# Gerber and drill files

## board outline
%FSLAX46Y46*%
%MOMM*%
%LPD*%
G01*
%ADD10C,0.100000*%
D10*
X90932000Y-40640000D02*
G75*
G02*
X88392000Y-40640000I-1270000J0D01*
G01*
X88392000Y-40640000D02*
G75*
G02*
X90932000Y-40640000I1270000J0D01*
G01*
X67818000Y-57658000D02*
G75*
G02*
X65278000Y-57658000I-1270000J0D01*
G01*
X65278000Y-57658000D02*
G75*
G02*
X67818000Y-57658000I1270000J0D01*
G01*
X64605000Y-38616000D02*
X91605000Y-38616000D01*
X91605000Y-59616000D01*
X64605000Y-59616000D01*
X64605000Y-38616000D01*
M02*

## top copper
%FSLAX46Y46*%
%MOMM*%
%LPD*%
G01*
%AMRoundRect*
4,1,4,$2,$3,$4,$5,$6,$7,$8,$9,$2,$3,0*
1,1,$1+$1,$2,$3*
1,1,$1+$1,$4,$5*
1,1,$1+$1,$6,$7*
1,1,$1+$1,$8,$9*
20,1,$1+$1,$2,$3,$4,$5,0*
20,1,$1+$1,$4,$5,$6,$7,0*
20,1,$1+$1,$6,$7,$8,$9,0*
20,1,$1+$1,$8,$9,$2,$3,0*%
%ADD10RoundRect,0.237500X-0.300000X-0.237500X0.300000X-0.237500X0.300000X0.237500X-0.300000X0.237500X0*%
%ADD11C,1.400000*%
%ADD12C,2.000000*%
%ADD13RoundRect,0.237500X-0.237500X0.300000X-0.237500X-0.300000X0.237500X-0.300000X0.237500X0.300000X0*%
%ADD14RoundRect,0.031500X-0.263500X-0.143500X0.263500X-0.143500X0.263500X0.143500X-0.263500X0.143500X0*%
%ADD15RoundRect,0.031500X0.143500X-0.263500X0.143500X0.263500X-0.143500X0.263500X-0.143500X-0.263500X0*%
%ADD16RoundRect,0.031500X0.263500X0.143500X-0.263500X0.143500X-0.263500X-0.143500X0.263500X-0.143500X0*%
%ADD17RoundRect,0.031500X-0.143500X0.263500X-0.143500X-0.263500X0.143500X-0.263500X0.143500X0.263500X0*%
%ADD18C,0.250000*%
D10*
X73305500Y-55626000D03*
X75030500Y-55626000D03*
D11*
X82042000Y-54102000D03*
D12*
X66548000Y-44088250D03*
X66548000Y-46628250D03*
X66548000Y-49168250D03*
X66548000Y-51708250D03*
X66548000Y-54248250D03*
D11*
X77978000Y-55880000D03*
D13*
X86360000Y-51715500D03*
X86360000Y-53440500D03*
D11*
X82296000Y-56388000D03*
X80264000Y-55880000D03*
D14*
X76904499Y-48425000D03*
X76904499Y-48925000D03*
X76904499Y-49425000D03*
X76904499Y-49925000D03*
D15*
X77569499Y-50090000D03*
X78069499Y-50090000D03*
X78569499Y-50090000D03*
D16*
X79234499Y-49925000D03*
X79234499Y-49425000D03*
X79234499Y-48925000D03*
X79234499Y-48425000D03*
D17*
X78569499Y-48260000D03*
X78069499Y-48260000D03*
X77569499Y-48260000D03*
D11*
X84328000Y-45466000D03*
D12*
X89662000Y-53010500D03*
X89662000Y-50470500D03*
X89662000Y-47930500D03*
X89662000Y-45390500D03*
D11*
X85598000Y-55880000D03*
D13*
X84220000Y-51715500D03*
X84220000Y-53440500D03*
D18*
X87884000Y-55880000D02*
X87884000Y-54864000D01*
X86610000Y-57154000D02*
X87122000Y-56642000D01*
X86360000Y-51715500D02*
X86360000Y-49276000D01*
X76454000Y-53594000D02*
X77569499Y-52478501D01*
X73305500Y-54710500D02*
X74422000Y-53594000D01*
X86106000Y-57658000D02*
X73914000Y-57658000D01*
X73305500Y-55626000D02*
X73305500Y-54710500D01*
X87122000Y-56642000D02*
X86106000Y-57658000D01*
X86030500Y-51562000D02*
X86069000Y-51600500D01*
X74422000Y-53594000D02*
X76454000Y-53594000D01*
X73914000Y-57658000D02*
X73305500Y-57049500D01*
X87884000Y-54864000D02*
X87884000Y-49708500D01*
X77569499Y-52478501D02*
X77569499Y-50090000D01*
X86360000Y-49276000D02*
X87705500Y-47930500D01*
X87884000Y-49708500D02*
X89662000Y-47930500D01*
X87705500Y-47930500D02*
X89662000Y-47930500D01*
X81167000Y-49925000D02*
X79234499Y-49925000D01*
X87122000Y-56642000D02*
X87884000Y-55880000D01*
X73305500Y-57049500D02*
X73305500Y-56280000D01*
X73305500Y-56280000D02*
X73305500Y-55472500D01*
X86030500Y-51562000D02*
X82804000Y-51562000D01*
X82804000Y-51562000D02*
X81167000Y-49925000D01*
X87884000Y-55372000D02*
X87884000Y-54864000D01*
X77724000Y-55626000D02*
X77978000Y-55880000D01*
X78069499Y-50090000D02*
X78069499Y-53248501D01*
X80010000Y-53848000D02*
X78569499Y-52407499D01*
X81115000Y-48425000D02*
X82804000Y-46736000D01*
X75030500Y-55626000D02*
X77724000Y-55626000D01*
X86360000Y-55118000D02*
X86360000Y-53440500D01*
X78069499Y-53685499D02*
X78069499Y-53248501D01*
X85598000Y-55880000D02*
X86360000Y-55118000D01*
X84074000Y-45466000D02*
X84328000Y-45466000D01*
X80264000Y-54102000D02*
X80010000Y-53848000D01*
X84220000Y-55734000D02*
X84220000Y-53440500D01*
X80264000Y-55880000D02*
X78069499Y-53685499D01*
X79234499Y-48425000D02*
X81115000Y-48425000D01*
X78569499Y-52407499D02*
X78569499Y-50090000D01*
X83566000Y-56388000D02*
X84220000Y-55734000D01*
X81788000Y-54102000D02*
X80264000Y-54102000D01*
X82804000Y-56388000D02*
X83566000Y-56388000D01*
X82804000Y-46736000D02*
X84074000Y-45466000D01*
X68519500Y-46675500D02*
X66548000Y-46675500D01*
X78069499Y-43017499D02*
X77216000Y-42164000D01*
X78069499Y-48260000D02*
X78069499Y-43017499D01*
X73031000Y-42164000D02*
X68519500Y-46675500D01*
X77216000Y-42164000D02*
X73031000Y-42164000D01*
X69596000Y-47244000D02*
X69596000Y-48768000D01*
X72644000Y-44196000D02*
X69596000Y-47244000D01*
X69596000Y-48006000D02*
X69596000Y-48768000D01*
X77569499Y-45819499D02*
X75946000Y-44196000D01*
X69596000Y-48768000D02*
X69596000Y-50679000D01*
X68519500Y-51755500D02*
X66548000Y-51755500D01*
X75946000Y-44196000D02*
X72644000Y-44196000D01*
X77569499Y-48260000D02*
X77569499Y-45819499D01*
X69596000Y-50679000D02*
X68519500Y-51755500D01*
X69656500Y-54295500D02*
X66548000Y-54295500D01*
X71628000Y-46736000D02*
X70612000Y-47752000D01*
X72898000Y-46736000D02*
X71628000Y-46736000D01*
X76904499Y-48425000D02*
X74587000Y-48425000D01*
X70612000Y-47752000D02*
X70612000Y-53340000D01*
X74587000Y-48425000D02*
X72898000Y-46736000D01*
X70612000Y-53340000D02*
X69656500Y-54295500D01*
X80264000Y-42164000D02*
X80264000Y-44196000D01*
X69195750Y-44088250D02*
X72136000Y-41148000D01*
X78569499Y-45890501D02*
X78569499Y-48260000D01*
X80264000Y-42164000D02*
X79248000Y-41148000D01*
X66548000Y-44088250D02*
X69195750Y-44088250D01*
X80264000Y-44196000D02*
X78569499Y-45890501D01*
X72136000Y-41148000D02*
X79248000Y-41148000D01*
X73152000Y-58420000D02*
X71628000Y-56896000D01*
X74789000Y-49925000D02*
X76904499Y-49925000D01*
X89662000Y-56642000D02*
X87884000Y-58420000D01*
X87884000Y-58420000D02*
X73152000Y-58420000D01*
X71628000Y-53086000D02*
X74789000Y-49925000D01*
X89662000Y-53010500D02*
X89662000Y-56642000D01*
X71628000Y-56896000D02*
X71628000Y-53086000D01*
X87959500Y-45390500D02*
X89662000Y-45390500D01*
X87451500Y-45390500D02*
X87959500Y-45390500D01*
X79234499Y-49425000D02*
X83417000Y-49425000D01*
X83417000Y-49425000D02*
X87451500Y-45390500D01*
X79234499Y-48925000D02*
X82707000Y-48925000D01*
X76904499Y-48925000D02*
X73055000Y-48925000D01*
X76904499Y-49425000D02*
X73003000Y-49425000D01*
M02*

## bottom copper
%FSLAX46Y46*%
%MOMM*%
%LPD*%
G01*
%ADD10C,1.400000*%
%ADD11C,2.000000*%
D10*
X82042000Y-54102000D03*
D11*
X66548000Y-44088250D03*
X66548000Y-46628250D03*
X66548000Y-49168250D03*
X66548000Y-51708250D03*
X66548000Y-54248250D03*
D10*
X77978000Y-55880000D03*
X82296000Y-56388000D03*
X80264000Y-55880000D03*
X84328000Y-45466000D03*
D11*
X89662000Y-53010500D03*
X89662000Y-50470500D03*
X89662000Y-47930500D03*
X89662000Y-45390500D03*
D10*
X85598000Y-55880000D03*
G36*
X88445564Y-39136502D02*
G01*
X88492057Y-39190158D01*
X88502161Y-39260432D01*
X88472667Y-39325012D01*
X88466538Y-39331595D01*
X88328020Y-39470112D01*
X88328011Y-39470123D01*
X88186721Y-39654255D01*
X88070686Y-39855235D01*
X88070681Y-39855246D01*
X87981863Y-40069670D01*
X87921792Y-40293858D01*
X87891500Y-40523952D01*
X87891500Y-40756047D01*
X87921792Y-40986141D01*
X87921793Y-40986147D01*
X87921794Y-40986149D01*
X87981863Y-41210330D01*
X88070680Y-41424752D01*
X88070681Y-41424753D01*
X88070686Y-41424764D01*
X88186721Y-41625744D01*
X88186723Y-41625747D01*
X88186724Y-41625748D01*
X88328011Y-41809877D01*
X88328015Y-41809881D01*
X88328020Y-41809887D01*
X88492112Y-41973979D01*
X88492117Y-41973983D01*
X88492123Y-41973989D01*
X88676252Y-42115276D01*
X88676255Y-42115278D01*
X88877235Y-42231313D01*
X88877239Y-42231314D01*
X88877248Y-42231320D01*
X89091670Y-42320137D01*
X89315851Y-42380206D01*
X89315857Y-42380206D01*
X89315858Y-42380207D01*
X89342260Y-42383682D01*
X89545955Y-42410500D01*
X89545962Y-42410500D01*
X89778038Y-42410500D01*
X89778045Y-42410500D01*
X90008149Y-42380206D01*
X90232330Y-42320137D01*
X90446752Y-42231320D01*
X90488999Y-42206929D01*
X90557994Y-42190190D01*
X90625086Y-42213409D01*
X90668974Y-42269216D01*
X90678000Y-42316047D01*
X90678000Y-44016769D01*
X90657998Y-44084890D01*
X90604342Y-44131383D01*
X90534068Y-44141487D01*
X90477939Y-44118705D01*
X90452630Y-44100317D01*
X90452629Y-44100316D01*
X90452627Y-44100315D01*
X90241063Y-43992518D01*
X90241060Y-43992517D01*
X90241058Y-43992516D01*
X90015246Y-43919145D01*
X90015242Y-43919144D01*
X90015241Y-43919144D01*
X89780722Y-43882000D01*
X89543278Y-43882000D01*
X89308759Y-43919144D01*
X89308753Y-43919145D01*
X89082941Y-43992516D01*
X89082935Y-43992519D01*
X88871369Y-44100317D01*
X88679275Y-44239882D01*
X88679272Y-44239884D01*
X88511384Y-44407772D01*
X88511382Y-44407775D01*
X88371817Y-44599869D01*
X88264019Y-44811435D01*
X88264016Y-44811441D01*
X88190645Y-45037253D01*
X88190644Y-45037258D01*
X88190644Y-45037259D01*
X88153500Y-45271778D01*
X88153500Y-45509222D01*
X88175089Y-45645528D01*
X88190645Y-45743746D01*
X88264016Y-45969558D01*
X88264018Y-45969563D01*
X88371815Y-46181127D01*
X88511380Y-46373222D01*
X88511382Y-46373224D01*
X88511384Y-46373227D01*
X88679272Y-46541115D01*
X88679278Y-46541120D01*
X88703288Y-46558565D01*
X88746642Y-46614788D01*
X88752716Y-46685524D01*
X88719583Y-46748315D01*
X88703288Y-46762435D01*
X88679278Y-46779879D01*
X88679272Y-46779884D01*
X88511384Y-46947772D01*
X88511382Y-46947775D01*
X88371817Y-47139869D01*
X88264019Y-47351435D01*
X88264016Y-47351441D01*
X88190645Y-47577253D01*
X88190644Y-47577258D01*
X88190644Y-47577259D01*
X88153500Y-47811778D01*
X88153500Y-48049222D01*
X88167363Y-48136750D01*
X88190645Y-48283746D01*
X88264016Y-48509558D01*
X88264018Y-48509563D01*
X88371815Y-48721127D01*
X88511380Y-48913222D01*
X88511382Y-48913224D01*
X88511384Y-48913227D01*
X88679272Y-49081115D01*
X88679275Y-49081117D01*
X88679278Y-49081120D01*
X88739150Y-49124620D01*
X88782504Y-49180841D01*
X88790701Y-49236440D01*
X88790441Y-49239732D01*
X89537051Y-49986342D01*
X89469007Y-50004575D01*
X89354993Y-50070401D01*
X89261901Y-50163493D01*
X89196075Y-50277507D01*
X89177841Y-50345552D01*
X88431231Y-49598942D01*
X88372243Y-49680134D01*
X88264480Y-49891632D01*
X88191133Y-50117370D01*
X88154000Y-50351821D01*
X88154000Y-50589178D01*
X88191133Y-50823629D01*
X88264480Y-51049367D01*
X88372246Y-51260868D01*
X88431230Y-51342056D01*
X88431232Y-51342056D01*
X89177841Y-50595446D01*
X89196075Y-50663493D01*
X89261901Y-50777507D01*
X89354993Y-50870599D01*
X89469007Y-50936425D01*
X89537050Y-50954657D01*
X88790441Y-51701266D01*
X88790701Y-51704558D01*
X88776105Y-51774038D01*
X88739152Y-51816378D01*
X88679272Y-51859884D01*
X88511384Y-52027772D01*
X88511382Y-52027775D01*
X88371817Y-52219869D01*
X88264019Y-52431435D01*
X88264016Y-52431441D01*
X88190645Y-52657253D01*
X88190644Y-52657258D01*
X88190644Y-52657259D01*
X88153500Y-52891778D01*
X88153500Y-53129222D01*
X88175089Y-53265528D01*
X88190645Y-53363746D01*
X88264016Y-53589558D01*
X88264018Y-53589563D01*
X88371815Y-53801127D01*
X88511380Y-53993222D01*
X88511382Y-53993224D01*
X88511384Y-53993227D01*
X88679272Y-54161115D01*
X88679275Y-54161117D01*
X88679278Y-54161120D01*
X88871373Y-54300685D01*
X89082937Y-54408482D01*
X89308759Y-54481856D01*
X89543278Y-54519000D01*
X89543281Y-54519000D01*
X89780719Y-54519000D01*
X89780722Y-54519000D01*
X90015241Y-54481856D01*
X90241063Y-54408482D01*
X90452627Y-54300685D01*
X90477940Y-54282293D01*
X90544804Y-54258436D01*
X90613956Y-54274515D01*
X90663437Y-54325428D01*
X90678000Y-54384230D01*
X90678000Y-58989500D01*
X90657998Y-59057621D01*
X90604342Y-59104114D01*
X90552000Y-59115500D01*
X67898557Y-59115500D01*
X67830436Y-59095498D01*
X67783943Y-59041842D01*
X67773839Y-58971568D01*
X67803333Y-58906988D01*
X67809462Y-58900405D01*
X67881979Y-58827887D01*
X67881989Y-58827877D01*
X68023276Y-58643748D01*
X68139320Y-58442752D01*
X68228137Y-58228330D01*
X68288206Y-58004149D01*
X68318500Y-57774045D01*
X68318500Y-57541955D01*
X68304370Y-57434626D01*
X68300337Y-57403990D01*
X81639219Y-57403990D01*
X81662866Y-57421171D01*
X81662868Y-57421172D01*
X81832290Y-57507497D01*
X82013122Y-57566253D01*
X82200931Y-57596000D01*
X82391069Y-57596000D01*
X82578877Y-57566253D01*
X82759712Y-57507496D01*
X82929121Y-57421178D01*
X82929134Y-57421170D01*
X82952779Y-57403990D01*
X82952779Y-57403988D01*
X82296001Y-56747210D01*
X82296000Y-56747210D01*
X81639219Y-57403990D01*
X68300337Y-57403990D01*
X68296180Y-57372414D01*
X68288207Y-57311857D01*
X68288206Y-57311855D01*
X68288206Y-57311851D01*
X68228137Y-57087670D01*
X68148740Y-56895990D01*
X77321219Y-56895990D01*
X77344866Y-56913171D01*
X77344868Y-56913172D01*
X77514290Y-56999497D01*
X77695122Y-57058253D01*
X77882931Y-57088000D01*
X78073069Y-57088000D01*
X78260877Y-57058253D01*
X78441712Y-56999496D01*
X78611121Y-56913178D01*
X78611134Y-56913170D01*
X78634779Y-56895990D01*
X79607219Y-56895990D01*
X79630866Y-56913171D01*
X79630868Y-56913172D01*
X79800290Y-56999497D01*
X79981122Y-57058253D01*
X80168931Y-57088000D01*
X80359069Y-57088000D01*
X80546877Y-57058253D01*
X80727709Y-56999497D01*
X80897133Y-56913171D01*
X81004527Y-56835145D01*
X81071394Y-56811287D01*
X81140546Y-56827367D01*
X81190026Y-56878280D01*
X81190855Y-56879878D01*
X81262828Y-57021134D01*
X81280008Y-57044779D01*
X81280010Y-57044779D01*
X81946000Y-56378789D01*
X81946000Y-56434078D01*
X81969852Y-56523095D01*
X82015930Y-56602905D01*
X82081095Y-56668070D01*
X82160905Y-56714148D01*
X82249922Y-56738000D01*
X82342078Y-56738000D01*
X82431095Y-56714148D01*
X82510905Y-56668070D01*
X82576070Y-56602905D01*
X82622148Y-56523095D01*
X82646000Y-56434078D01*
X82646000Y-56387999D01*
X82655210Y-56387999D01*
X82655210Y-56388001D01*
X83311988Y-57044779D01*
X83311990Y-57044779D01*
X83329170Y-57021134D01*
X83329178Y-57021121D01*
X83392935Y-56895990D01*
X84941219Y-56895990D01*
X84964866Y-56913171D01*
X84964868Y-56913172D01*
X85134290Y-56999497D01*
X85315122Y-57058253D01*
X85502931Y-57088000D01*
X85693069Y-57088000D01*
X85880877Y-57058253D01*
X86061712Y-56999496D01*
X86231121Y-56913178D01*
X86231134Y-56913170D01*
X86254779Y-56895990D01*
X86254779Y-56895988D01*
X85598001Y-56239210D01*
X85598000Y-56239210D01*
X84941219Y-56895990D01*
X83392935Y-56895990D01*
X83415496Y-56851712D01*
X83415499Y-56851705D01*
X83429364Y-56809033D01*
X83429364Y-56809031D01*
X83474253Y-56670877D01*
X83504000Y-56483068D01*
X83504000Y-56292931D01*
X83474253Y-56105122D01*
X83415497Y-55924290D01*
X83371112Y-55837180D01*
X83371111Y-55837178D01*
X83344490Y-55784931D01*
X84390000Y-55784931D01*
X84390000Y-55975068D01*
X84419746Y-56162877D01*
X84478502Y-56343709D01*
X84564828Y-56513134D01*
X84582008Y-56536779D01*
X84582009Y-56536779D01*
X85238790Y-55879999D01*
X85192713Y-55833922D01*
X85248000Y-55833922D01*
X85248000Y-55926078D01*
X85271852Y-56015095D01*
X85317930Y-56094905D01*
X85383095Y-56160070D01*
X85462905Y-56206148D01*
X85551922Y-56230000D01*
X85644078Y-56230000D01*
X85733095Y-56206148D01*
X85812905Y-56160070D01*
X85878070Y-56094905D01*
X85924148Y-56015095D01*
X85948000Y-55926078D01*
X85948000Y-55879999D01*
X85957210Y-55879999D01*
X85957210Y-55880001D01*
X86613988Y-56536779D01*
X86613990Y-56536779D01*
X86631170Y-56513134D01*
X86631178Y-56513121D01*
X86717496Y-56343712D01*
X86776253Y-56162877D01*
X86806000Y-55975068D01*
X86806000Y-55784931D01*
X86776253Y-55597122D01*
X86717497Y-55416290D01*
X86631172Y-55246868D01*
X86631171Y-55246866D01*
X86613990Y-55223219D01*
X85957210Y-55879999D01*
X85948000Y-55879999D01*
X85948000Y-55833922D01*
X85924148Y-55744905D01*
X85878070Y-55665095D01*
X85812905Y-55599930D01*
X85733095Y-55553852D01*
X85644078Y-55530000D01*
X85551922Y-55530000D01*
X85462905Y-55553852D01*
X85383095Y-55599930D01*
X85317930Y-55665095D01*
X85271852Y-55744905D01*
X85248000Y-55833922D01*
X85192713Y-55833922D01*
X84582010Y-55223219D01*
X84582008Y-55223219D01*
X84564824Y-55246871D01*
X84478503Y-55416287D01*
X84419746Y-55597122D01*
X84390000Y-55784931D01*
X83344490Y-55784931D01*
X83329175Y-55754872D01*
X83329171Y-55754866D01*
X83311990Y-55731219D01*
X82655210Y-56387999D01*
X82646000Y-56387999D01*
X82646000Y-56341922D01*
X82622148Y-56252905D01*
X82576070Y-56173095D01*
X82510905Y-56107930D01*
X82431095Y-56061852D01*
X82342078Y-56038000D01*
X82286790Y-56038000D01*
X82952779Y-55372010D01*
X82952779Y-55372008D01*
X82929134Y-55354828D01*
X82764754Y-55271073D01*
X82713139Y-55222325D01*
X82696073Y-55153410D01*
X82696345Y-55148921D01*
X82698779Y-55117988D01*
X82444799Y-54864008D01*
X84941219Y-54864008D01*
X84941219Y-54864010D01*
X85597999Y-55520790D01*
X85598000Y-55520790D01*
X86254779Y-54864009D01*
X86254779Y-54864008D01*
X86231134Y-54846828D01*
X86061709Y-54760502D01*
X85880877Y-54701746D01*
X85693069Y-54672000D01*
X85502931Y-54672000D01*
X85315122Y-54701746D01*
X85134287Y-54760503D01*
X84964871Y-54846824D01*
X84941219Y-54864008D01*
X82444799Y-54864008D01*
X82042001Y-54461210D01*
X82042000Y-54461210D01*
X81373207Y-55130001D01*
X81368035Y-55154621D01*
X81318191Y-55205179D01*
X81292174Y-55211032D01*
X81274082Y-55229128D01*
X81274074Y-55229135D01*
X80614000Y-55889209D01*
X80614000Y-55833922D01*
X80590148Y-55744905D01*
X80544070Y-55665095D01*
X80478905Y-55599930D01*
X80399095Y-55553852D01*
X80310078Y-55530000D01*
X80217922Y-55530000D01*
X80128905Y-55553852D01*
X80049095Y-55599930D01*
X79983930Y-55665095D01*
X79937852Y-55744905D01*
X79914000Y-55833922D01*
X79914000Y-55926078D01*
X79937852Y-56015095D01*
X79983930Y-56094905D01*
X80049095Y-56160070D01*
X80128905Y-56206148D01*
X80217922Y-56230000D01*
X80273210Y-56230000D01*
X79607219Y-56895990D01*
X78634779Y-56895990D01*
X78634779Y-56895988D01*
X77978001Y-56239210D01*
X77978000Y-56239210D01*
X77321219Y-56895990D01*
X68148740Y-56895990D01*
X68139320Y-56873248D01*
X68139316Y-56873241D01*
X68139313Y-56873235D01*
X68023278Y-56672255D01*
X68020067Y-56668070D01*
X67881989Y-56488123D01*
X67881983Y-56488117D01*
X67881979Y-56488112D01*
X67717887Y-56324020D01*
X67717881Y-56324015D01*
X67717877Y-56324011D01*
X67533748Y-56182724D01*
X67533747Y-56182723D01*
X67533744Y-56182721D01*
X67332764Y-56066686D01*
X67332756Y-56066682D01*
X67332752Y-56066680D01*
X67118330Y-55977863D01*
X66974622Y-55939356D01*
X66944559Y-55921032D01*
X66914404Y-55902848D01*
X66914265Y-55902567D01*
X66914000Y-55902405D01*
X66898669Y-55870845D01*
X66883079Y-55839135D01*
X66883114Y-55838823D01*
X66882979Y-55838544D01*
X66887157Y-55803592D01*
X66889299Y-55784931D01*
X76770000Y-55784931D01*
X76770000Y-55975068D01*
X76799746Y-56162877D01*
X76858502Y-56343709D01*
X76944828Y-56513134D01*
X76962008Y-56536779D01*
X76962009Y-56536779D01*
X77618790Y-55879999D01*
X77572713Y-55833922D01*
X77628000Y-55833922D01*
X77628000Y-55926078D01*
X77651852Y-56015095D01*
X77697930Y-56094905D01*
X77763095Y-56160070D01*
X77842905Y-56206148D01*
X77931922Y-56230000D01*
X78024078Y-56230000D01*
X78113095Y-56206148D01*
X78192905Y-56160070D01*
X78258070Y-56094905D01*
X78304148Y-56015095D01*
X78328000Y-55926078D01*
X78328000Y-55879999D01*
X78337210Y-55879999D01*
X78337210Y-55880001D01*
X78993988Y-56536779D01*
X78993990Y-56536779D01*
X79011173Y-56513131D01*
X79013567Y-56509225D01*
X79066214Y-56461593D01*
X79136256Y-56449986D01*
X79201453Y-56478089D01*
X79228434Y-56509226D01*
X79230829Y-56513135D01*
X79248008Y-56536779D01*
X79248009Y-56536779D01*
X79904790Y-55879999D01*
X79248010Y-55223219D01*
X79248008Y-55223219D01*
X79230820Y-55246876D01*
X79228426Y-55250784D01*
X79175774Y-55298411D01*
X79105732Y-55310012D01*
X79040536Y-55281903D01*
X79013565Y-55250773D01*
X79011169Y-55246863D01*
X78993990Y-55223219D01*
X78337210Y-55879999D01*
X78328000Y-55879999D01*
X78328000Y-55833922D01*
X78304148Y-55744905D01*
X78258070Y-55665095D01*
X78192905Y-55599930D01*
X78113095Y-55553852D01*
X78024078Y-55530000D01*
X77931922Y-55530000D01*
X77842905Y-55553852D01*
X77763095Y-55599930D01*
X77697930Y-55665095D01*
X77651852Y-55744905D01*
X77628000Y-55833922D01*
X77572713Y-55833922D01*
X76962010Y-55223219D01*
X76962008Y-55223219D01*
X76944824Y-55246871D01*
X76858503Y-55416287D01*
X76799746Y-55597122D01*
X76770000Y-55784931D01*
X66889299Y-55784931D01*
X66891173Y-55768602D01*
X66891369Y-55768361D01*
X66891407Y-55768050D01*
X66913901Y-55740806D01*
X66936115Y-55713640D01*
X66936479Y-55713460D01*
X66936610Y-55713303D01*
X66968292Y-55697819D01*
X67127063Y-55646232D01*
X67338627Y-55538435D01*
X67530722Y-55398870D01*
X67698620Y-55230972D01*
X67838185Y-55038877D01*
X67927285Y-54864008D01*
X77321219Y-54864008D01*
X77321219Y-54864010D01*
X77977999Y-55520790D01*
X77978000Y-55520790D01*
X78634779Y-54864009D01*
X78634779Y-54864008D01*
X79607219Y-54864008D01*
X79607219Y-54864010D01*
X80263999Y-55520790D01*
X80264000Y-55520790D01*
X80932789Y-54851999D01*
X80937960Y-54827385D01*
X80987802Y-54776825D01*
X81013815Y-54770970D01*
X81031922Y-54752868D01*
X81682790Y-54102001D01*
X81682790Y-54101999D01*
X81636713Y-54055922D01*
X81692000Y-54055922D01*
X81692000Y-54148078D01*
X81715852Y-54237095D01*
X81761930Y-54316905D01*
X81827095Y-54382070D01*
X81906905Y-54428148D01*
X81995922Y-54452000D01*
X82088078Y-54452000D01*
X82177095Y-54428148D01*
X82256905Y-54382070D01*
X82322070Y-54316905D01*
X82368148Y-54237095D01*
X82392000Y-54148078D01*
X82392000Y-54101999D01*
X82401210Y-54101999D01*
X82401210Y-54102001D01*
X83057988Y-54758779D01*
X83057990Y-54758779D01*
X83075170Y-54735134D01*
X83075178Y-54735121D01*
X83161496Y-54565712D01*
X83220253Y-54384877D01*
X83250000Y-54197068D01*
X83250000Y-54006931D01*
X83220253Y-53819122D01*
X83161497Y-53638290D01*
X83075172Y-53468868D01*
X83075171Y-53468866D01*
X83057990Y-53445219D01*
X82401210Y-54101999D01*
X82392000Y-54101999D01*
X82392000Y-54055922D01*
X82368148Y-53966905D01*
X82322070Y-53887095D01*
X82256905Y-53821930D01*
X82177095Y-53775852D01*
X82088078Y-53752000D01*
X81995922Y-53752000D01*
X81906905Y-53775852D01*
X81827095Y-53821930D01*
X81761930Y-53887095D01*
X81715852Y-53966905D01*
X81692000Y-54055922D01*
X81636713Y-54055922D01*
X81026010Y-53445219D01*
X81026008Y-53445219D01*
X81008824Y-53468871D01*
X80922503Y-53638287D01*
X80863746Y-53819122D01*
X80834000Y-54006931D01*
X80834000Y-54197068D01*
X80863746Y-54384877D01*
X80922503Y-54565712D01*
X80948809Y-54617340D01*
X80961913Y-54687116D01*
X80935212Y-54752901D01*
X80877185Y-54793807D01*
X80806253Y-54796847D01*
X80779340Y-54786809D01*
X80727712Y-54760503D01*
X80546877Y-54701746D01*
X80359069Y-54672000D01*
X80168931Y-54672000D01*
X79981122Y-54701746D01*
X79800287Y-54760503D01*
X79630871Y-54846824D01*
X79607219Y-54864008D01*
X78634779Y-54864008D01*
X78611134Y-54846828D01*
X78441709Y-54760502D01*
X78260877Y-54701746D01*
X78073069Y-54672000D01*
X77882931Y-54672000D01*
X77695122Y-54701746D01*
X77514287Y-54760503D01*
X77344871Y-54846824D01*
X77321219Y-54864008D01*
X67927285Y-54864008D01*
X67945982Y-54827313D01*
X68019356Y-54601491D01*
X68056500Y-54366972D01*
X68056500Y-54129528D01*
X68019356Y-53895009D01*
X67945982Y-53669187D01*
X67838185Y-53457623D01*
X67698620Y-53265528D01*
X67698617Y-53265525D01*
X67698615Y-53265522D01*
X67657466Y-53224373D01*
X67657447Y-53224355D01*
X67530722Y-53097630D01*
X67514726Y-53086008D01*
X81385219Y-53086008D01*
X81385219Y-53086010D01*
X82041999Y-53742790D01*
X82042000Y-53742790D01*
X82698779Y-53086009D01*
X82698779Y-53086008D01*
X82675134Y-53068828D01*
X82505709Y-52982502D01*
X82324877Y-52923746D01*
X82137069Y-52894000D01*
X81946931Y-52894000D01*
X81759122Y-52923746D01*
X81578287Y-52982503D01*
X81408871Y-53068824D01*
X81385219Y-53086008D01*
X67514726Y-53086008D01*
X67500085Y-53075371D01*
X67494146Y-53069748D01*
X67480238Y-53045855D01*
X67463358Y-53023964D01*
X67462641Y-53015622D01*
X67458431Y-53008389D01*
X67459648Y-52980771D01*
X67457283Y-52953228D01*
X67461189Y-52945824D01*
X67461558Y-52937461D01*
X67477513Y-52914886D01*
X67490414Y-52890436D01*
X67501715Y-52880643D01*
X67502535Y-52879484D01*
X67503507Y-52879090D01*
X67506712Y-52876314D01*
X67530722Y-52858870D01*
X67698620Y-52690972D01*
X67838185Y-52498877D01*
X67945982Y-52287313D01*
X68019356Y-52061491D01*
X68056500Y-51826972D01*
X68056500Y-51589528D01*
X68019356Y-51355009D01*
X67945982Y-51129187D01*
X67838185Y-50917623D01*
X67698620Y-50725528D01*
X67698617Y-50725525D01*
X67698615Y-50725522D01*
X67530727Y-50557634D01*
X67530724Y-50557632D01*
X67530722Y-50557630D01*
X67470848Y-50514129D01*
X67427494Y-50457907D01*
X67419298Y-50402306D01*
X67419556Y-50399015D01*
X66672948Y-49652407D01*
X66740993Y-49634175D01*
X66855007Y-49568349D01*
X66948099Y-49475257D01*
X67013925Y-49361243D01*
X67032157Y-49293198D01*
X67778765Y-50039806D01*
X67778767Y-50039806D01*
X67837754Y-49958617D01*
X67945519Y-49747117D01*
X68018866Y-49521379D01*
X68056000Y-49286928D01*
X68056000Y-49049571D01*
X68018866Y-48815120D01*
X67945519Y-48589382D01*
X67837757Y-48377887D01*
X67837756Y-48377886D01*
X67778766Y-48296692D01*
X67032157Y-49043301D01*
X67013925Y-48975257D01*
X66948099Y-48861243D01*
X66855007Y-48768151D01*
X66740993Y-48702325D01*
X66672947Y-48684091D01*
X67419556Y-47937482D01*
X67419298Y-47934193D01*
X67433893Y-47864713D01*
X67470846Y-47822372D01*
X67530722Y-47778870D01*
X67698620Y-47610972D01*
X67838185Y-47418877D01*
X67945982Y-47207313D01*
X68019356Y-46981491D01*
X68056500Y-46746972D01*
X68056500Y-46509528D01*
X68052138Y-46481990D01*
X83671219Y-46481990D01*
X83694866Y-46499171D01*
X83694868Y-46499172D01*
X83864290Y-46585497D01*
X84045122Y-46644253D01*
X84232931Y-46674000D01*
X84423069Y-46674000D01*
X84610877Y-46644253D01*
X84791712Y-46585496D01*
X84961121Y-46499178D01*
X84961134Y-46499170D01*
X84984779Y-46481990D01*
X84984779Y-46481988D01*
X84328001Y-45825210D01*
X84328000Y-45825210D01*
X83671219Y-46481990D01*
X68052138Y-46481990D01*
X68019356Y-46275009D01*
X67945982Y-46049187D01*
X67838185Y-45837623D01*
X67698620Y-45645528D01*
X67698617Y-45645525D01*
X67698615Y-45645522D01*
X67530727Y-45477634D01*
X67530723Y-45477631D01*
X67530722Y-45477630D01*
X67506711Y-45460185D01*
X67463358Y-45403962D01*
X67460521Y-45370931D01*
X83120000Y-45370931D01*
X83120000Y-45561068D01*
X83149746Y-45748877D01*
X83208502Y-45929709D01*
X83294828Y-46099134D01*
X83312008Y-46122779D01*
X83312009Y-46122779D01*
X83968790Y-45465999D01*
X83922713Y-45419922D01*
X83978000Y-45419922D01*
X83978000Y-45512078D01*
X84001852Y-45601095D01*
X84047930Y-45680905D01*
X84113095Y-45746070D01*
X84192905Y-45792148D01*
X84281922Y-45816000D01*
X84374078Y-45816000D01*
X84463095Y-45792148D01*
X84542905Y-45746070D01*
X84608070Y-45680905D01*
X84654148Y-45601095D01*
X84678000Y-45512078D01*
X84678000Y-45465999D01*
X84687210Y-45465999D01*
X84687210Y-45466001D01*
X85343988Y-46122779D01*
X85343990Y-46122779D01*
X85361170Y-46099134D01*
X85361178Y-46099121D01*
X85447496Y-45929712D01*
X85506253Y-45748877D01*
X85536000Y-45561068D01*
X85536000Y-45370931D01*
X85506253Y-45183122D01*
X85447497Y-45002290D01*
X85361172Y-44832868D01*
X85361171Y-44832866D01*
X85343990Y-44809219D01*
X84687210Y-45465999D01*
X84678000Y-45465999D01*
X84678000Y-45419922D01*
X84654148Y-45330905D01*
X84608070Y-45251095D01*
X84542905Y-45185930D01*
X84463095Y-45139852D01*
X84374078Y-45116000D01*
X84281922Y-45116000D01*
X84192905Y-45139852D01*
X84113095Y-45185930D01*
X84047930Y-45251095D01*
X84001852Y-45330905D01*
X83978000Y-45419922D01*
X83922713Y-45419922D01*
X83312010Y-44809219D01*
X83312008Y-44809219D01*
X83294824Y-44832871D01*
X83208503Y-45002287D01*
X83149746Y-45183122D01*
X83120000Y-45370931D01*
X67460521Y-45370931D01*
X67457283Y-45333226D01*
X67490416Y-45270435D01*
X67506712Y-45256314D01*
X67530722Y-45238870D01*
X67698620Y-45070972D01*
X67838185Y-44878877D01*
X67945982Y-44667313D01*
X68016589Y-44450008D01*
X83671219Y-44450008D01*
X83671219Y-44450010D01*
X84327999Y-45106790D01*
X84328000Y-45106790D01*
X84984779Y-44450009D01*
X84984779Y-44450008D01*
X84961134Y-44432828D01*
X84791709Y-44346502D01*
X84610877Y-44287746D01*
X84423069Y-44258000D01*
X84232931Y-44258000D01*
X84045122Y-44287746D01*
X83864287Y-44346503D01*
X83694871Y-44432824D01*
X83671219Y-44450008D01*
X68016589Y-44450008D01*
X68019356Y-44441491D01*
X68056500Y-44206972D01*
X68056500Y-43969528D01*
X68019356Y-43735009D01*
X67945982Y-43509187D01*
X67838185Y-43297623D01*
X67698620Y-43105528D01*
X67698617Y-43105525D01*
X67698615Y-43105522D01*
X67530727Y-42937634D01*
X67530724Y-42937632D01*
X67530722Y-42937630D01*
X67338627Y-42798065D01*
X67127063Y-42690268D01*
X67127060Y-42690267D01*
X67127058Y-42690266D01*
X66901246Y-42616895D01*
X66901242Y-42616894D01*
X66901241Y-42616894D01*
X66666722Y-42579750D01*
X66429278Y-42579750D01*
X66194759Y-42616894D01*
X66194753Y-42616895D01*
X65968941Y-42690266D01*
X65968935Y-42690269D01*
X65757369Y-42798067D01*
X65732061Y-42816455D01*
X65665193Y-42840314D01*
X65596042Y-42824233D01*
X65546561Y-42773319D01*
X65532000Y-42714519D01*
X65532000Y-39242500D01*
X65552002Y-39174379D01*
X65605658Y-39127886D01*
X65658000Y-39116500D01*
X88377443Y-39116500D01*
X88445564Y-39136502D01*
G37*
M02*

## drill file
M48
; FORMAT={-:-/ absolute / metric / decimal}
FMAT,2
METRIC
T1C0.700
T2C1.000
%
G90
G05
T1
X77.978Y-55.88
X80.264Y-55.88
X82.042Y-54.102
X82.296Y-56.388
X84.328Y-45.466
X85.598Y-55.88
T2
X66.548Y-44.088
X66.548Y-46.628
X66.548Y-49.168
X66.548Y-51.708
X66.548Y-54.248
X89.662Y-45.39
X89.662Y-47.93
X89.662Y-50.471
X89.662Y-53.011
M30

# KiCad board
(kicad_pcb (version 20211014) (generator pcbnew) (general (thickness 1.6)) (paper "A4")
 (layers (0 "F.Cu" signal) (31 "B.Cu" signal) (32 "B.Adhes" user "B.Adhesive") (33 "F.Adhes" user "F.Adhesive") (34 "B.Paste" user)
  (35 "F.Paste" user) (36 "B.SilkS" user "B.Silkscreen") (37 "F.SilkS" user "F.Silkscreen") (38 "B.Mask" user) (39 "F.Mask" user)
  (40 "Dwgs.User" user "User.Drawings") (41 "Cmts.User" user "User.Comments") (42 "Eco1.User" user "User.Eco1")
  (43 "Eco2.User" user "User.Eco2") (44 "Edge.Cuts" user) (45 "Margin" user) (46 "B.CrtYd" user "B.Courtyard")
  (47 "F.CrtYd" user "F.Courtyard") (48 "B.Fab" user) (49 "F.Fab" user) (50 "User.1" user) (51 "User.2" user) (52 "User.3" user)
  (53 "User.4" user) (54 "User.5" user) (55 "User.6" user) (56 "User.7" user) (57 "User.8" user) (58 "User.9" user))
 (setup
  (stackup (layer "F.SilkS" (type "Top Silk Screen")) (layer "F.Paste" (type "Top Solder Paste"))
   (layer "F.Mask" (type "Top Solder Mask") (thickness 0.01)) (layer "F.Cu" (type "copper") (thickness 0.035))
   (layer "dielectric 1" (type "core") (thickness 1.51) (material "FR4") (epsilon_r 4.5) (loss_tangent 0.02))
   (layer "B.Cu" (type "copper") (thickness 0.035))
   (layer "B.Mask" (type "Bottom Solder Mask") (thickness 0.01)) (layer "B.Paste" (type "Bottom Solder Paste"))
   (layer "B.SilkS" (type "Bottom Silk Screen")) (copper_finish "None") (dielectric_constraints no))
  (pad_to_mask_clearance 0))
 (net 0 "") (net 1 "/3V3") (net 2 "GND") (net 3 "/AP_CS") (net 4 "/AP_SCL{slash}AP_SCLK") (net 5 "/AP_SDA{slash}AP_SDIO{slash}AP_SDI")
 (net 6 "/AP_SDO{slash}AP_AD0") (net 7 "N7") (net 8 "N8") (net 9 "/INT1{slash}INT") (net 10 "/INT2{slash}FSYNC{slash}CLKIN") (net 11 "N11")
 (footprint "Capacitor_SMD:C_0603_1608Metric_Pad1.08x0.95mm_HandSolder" (layer "F.Cu") (at 74.168 55.626)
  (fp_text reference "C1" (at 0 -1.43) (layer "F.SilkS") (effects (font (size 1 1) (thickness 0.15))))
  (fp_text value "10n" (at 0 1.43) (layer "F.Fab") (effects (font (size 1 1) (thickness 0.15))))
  (pad "1" smd roundrect (at -0.8625 0) (size 1.075 0.95) (layers "F.Cu" "F.Paste" "F.Mask") (roundrect_rratio 0.25) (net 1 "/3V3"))
  (pad "2" smd roundrect (at 0.8625 0) (size 1.075 0.95) (layers "F.Cu" "F.Paste" "F.Mask") (roundrect_rratio 0.25) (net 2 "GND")))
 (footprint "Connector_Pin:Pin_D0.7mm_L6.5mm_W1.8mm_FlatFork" (layer "F.Cu") (at 82.042 54.102)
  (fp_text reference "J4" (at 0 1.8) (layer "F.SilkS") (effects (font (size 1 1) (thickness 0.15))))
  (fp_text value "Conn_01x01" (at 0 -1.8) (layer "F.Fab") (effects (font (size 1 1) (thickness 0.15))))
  (pad "1" thru_hole circle (at 0 0) (size 1.4 1.4) (drill 0.7) (layers *.Cu *.Mask) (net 2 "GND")))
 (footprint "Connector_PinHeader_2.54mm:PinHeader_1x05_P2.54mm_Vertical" (layer "F.Cu") (at 66.548 44.08825)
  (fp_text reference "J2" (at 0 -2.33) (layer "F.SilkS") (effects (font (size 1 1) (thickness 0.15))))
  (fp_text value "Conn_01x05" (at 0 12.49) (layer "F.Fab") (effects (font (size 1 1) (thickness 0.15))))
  (pad "1" thru_hole circle (at 0 0) (size 2 2) (drill 1) (layers *.Cu *.Mask) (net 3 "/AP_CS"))
  (pad "2" thru_hole circle (at 0 2.54) (size 2 2) (drill 1) (layers *.Cu *.Mask) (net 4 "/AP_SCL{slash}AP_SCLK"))
  (pad "3" thru_hole circle (at 0 5.08) (size 2 2) (drill 1) (layers *.Cu *.Mask) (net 2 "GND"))
  (pad "4" thru_hole circle (at 0 7.62) (size 2 2) (drill 1) (layers *.Cu *.Mask) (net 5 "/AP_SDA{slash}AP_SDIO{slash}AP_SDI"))
  (pad "5" thru_hole circle (at 0 10.16) (size 2 2) (drill 1) (layers *.Cu *.Mask) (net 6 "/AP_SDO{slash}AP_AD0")))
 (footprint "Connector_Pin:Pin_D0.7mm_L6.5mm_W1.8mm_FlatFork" (layer "F.Cu") (at 77.978 55.88)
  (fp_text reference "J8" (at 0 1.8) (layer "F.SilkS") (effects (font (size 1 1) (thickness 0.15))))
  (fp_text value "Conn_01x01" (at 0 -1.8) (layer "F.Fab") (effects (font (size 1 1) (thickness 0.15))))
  (pad "1" thru_hole circle (at 0 0) (size 1.4 1.4) (drill 0.7) (layers *.Cu *.Mask) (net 2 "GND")))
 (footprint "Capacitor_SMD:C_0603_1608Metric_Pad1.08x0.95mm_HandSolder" (layer "F.Cu") (at 86.36 52.578 -90)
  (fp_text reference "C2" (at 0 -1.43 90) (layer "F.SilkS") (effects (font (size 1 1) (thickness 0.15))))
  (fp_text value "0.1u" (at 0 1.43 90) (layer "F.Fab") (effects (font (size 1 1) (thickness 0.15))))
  (pad "1" smd roundrect (at -0.8625 0 270) (size 1.075 0.95) (layers "F.Cu" "F.Paste" "F.Mask") (roundrect_rratio 0.25) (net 1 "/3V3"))
  (pad "2" smd roundrect (at 0.8625 0 270) (size 1.075 0.95) (layers "F.Cu" "F.Paste" "F.Mask") (roundrect_rratio 0.25) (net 2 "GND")))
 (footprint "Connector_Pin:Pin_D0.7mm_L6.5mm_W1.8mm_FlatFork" (layer "F.Cu") (at 82.296 56.388)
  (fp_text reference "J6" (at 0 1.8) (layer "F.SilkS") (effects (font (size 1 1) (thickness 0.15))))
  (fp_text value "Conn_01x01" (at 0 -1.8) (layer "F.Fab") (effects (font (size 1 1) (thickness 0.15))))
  (pad "1" thru_hole circle (at 0 0) (size 1.4 1.4) (drill 0.7) (layers *.Cu *.Mask) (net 2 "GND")))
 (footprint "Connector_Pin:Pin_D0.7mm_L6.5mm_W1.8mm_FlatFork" (layer "F.Cu") (at 80.264 55.88)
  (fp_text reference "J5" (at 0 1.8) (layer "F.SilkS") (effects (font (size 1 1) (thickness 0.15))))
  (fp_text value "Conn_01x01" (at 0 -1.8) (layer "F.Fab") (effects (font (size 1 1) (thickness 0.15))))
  (pad "1" thru_hole circle (at 0 0) (size 1.4 1.4) (drill 0.7) (layers *.Cu *.Mask) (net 2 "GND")))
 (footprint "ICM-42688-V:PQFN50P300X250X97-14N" (layer "F.Cu") (at 78.069499 49.175)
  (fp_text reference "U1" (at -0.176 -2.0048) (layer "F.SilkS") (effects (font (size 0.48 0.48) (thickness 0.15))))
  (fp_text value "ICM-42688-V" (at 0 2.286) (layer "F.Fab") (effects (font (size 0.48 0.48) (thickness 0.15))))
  (pad "1" smd roundrect locked (at -1.165 -0.75) (size 0.59 0.35) (layers "F.Cu" "F.Paste") (roundrect_rratio 0.09)
   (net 6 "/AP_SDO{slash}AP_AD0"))
  (pad "2" smd roundrect locked (at -1.165 -0.25) (size 0.59 0.35) (layers "F.Cu" "F.Paste") (roundrect_rratio 0.09) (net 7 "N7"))
  (pad "3" smd roundrect locked (at -1.165 0.25) (size 0.59 0.35) (layers "F.Cu" "F.Paste") (roundrect_rratio 0.09) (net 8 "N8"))
  (pad "4" smd roundrect locked (at -1.165 0.75) (size 0.59 0.35) (layers "F.Cu" "F.Paste") (roundrect_rratio 0.09)
   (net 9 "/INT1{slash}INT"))
  (pad "5" smd roundrect locked (at -0.5 0.915 90) (size 0.59 0.35) (layers "F.Cu" "F.Paste") (roundrect_rratio 0.09) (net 1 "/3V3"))
  (pad "6" smd roundrect locked (at 0 0.915 90) (size 0.59 0.35) (layers "F.Cu" "F.Paste") (roundrect_rratio 0.09) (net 2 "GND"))
  (pad "7" smd roundrect locked (at 0.5 0.915 90) (size 0.59 0.35) (layers "F.Cu" "F.Paste") (roundrect_rratio 0.09) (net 2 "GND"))
  (pad "8" smd roundrect locked (at 1.165 0.75 180) (size 0.59 0.35) (layers "F.Cu" "F.Paste") (roundrect_rratio 0.09) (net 1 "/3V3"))
  (pad "9" smd roundrect locked (at 1.165 0.25 180) (size 0.59 0.35) (layers "F.Cu" "F.Paste") (roundrect_rratio 0.09)
   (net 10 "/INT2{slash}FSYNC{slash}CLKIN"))
  (pad "10" smd roundrect locked (at 1.165 -0.25 180) (size 0.59 0.35) (layers "F.Cu" "F.Paste") (roundrect_rratio 0.09) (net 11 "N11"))
  (pad "11" smd roundrect locked (at 1.165 -0.75 180) (size 0.59 0.35) (layers "F.Cu" "F.Paste") (roundrect_rratio 0.09) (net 2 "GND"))
  (pad "12" smd roundrect locked (at 0.5 -0.915 270) (size 0.59 0.35) (layers "F.Cu" "F.Paste") (roundrect_rratio 0.09) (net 3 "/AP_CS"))
  (pad "13" smd roundrect locked (at 0 -0.915 270) (size 0.59 0.35) (layers "F.Cu" "F.Paste") (roundrect_rratio 0.09)
   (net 4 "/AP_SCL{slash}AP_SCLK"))
  (pad "14" smd roundrect locked (at -0.5 -0.915 270) (size 0.59 0.35) (layers "F.Cu" "F.Paste") (roundrect_rratio 0.09)
   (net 5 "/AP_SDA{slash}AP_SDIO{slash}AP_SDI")))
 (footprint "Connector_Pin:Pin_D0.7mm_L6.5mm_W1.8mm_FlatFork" (layer "F.Cu") (at 84.328 45.466)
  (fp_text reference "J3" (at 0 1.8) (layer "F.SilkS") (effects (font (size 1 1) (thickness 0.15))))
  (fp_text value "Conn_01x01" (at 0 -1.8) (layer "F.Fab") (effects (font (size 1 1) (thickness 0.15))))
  (pad "1" thru_hole circle (at 0 0) (size 1.4 1.4) (drill 0.7) (layers *.Cu *.Mask) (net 2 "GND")))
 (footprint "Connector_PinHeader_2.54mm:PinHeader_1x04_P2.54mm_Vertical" (layer "F.Cu") (at 89.662 53.0105 180)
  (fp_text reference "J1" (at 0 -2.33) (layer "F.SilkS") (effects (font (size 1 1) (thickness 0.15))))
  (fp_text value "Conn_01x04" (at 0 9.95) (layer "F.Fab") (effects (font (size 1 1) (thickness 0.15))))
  (pad "1" thru_hole circle (at 0 0 180) (size 2 2) (drill 1) (layers *.Cu *.Mask) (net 9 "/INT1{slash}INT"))
  (pad "2" thru_hole circle (at 0 2.54 180) (size 2 2) (drill 1) (layers *.Cu *.Mask) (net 2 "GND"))
  (pad "3" thru_hole circle (at 0 5.08 180) (size 2 2) (drill 1) (layers *.Cu *.Mask) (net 1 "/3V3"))
  (pad "4" thru_hole circle (at 0 7.62 180) (size 2 2) (drill 1) (layers *.Cu *.Mask) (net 10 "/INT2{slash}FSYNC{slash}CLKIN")))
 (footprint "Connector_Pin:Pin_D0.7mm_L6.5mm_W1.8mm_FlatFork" (layer "F.Cu") (at 85.598 55.88)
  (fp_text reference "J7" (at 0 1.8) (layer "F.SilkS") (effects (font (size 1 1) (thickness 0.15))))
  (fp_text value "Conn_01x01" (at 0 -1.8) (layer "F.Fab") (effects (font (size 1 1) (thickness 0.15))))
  (pad "1" thru_hole circle (at 0 0) (size 1.4 1.4) (drill 0.7) (layers *.Cu *.Mask) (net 2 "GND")))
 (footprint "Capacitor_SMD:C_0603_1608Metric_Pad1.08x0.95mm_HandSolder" (layer "F.Cu") (at 84.22 52.578 -90)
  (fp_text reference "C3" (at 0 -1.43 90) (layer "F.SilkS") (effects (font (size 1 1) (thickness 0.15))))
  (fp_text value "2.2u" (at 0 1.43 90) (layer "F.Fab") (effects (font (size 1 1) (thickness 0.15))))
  (pad "1" smd roundrect (at -0.8625 0 270) (size 1.075 0.95) (layers "F.Cu" "F.Paste" "F.Mask") (roundrect_rratio 0.25) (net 1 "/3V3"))
  (pad "2" smd roundrect (at 0.8625 0 270) (size 1.075 0.95) (layers "F.Cu" "F.Paste" "F.Mask") (roundrect_rratio 0.25) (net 2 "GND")))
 (gr_circle (center 89.662 40.64) (end 90.932 40.64) (layer "Edge.Cuts") (width 0.1) (fill none))
 (gr_circle (center 66.548 57.658) (end 67.818 57.658) (layer "Edge.Cuts") (width 0.1) (fill none))
 (gr_rect (start 64.605 38.616) (end 91.605 59.616) (layer "Edge.Cuts") (width 0.1) (fill none))
 (segment (start 87.884 55.88) (end 87.884 54.864) (width 0.25) (layer "F.Cu") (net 1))
 (segment (start 86.61 57.154) (end 87.122 56.642) (width 0.25) (layer "F.Cu") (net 1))
 (segment (start 86.36 51.7155) (end 86.36 49.276) (width 0.25) (layer "F.Cu") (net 1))
 (segment (start 76.454 53.594) (end 77.569499 52.478501) (width 0.25) (layer "F.Cu") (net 1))
 (segment (start 73.3055 54.7105) (end 74.422 53.594) (width 0.25) (layer "F.Cu") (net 1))
 (segment (start 86.106 57.658) (end 73.914 57.658) (width 0.25) (layer "F.Cu") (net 1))
 (segment (start 73.3055 55.626) (end 73.3055 54.7105) (width 0.25) (layer "F.Cu") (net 1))
 (segment (start 87.122 56.642) (end 86.106 57.658) (width 0.25) (layer "F.Cu") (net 1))
 (segment (start 86.0305 51.562) (end 86.069 51.6005) (width 0.25) (layer "F.Cu") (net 1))
 (segment (start 74.422 53.594) (end 76.454 53.594) (width 0.25) (layer "F.Cu") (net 1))
 (segment (start 73.914 57.658) (end 73.3055 57.0495) (width 0.25) (layer "F.Cu") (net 1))
 (segment (start 87.884 54.864) (end 87.884 49.7085) (width 0.25) (layer "F.Cu") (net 1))
 (segment (start 77.569499 52.478501) (end 77.569499 50.09) (width 0.25) (layer "F.Cu") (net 1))
 (segment (start 86.36 49.276) (end 87.7055 47.9305) (width 0.25) (layer "F.Cu") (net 1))
 (segment (start 87.884 49.7085) (end 89.662 47.9305) (width 0.25) (layer "F.Cu") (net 1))
 (segment (start 87.7055 47.9305) (end 89.662 47.9305) (width 0.25) (layer "F.Cu") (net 1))
 (segment (start 81.167 49.925) (end 79.234499 49.925) (width 0.25) (layer "F.Cu") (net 1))
 (segment (start 87.122 56.642) (end 87.884 55.88) (width 0.25) (layer "F.Cu") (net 1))
 (segment (start 73.3055 57.0495) (end 73.3055 56.28) (width 0.25) (layer "F.Cu") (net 1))
 (segment (start 73.3055 56.28) (end 73.3055 55.4725) (width 0.25) (layer "F.Cu") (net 1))
 (segment (start 86.0305 51.562) (end 82.804 51.562) (width 0.25) (layer "F.Cu") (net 1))
 (segment (start 82.804 51.562) (end 81.167 49.925) (width 0.25) (layer "F.Cu") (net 1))
 (segment (start 87.884 55.372) (end 87.884 54.864) (width 0.25) (layer "F.Cu") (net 1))
 (segment (start 77.724 55.626) (end 77.978 55.88) (width 0.25) (layer "F.Cu") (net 2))
 (segment (start 78.069499 50.09) (end 78.069499 53.248501) (width 0.25) (layer "F.Cu") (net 2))
 (segment (start 80.01 53.848) (end 78.569499 52.407499) (width 0.25) (layer "F.Cu") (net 2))
 (segment (start 81.115 48.425) (end 82.804 46.736) (width 0.25) (layer "F.Cu") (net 2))
 (segment (start 75.0305 55.626) (end 77.724 55.626) (width 0.25) (layer "F.Cu") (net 2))
 (segment (start 86.36 55.118) (end 86.36 53.4405) (width 0.25) (layer "F.Cu") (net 2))
 (segment (start 78.069499 53.685499) (end 78.069499 53.248501) (width 0.25) (layer "F.Cu") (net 2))
 (segment (start 85.598 55.88) (end 86.36 55.118) (width 0.25) (layer "F.Cu") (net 2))
 (segment (start 84.074 45.466) (end 84.328 45.466) (width 0.25) (layer "F.Cu") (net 2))
 (segment (start 80.264 54.102) (end 80.01 53.848) (width 0.25) (layer "F.Cu") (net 2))
 (segment (start 84.22 55.734) (end 84.22 53.4405) (width 0.25) (layer "F.Cu") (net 2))
 (segment (start 80.264 55.88) (end 78.069499 53.685499) (width 0.25) (layer "F.Cu") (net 2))
 (segment (start 79.234499 48.425) (end 81.115 48.425) (width 0.25) (layer "F.Cu") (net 2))
 (segment (start 78.569499 52.407499) (end 78.569499 50.09) (width 0.25) (layer "F.Cu") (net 2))
 (segment (start 83.566 56.388) (end 84.22 55.734) (width 0.25) (layer "F.Cu") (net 2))
 (segment (start 81.788 54.102) (end 80.264 54.102) (width 0.25) (layer "F.Cu") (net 2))
 (segment (start 82.804 56.388) (end 83.566 56.388) (width 0.25) (layer "F.Cu") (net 2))
 (segment (start 82.804 46.736) (end 84.074 45.466) (width 0.25) (layer "F.Cu") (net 2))
 (segment (start 68.5195 46.6755) (end 66.548 46.6755) (width 0.25) (layer "F.Cu") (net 4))
 (segment (start 78.069499 43.017499) (end 77.216 42.164) (width 0.25) (layer "F.Cu") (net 4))
 (segment (start 78.069499 48.26) (end 78.069499 43.017499) (width 0.25) (layer "F.Cu") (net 4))
 (segment (start 73.031 42.164) (end 68.5195 46.6755) (width 0.25) (layer "F.Cu") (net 4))
 (segment (start 77.216 42.164) (end 73.031 42.164) (width 0.25) (layer "F.Cu") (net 4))
 (segment (start 69.596 47.244) (end 69.596 48.768) (width 0.25) (layer "F.Cu") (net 5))
 (segment (start 72.644 44.196) (end 69.596 47.244) (width 0.25) (layer "F.Cu") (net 5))
 (segment (start 69.596 48.006) (end 69.596 48.768) (width 0.25) (layer "F.Cu") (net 5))
 (segment (start 77.569499 45.819499) (end 75.946 44.196) (width 0.25) (layer "F.Cu") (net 5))
 (segment (start 69.596 48.768) (end 69.596 50.679) (width 0.25) (layer "F.Cu") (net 5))
 (segment (start 68.5195 51.7555) (end 66.548 51.7555) (width 0.25) (layer "F.Cu") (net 5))
 (segment (start 75.946 44.196) (end 72.644 44.196) (width 0.25) (layer "F.Cu") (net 5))
 (segment (start 77.569499 48.26) (end 77.569499 45.819499) (width 0.25) (layer "F.Cu") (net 5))
 (segment (start 69.596 50.679) (end 68.5195 51.7555) (width 0.25) (layer "F.Cu") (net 5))
 (segment (start 69.6565 54.2955) (end 66.548 54.2955) (width 0.25) (layer "F.Cu") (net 6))
 (segment (start 71.628 46.736) (end 70.612 47.752) (width 0.25) (layer "F.Cu") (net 6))
 (segment (start 72.898 46.736) (end 71.628 46.736) (width 0.25) (layer "F.Cu") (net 6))
 (segment (start 76.904499 48.425) (end 74.587 48.425) (width 0.25) (layer "F.Cu") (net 6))
 (segment (start 70.612 47.752) (end 70.612 53.34) (width 0.25) (layer "F.Cu") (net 6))
 (segment (start 74.587 48.425) (end 72.898 46.736) (width 0.25) (layer "F.Cu") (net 6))
 (segment (start 70.612 53.34) (end 69.6565 54.2955) (width 0.25) (layer "F.Cu") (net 6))
 (segment (start 80.264 42.164) (end 80.264 44.196) (width 0.25) (layer "F.Cu") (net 3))
 (segment (start 69.19575 44.08825) (end 72.136 41.148) (width 0.25) (layer "F.Cu") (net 3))
 (segment (start 78.569499 45.890501) (end 78.569499 48.26) (width 0.25) (layer "F.Cu") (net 3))
 (segment (start 80.264 42.164) (end 79.248 41.148) (width 0.25) (layer "F.Cu") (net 3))
 (segment (start 66.548 44.08825) (end 69.19575 44.08825) (width 0.25) (layer "F.Cu") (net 3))
 (segment (start 80.264 44.196) (end 78.569499 45.890501) (width 0.25) (layer "F.Cu") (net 3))
 (segment (start 72.136 41.148) (end 79.248 41.148) (width 0.25) (layer "F.Cu") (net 3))
 (segment (start 73.152 58.42) (end 71.628 56.896) (width 0.25) (layer "F.Cu") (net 9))
 (segment (start 74.789 49.925) (end 76.904499 49.925) (width 0.25) (layer "F.Cu") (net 9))
 (segment (start 89.662 56.642) (end 87.884 58.42) (width 0.25) (layer "F.Cu") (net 9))
 (segment (start 87.884 58.42) (end 73.152 58.42) (width 0.25) (layer "F.Cu") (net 9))
 (segment (start 71.628 53.086) (end 74.789 49.925) (width 0.25) (layer "F.Cu") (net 9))
 (segment (start 89.662 53.0105) (end 89.662 56.642) (width 0.25) (layer "F.Cu") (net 9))
 (segment (start 71.628 56.896) (end 71.628 53.086) (width 0.25) (layer "F.Cu") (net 9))
 (segment (start 87.9595 45.3905) (end 89.662 45.3905) (width 0.25) (layer "F.Cu") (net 10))
 (segment (start 87.4515 45.3905) (end 87.9595 45.3905) (width 0.25) (layer "F.Cu") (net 10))
 (segment (start 79.234499 49.425) (end 83.417 49.425) (width 0.25) (layer "F.Cu") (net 10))
 (segment (start 83.417 49.425) (end 87.4515 45.3905) (width 0.25) (layer "F.Cu") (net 10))
 (segment (start 79.234499 48.925) (end 82.707 48.925) (width 0.25) (layer "F.Cu") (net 11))
 (segment (start 76.904499 48.925) (end 73.055 48.925) (width 0.25) (layer "F.Cu") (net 7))
 (segment (start 76.904499 49.425) (end 73.003 49.425) (width 0.25) (layer "F.Cu") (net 8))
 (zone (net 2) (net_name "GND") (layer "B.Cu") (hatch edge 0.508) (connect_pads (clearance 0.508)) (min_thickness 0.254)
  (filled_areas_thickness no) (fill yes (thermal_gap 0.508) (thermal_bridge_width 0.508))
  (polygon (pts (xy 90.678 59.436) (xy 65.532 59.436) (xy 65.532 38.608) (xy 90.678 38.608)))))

